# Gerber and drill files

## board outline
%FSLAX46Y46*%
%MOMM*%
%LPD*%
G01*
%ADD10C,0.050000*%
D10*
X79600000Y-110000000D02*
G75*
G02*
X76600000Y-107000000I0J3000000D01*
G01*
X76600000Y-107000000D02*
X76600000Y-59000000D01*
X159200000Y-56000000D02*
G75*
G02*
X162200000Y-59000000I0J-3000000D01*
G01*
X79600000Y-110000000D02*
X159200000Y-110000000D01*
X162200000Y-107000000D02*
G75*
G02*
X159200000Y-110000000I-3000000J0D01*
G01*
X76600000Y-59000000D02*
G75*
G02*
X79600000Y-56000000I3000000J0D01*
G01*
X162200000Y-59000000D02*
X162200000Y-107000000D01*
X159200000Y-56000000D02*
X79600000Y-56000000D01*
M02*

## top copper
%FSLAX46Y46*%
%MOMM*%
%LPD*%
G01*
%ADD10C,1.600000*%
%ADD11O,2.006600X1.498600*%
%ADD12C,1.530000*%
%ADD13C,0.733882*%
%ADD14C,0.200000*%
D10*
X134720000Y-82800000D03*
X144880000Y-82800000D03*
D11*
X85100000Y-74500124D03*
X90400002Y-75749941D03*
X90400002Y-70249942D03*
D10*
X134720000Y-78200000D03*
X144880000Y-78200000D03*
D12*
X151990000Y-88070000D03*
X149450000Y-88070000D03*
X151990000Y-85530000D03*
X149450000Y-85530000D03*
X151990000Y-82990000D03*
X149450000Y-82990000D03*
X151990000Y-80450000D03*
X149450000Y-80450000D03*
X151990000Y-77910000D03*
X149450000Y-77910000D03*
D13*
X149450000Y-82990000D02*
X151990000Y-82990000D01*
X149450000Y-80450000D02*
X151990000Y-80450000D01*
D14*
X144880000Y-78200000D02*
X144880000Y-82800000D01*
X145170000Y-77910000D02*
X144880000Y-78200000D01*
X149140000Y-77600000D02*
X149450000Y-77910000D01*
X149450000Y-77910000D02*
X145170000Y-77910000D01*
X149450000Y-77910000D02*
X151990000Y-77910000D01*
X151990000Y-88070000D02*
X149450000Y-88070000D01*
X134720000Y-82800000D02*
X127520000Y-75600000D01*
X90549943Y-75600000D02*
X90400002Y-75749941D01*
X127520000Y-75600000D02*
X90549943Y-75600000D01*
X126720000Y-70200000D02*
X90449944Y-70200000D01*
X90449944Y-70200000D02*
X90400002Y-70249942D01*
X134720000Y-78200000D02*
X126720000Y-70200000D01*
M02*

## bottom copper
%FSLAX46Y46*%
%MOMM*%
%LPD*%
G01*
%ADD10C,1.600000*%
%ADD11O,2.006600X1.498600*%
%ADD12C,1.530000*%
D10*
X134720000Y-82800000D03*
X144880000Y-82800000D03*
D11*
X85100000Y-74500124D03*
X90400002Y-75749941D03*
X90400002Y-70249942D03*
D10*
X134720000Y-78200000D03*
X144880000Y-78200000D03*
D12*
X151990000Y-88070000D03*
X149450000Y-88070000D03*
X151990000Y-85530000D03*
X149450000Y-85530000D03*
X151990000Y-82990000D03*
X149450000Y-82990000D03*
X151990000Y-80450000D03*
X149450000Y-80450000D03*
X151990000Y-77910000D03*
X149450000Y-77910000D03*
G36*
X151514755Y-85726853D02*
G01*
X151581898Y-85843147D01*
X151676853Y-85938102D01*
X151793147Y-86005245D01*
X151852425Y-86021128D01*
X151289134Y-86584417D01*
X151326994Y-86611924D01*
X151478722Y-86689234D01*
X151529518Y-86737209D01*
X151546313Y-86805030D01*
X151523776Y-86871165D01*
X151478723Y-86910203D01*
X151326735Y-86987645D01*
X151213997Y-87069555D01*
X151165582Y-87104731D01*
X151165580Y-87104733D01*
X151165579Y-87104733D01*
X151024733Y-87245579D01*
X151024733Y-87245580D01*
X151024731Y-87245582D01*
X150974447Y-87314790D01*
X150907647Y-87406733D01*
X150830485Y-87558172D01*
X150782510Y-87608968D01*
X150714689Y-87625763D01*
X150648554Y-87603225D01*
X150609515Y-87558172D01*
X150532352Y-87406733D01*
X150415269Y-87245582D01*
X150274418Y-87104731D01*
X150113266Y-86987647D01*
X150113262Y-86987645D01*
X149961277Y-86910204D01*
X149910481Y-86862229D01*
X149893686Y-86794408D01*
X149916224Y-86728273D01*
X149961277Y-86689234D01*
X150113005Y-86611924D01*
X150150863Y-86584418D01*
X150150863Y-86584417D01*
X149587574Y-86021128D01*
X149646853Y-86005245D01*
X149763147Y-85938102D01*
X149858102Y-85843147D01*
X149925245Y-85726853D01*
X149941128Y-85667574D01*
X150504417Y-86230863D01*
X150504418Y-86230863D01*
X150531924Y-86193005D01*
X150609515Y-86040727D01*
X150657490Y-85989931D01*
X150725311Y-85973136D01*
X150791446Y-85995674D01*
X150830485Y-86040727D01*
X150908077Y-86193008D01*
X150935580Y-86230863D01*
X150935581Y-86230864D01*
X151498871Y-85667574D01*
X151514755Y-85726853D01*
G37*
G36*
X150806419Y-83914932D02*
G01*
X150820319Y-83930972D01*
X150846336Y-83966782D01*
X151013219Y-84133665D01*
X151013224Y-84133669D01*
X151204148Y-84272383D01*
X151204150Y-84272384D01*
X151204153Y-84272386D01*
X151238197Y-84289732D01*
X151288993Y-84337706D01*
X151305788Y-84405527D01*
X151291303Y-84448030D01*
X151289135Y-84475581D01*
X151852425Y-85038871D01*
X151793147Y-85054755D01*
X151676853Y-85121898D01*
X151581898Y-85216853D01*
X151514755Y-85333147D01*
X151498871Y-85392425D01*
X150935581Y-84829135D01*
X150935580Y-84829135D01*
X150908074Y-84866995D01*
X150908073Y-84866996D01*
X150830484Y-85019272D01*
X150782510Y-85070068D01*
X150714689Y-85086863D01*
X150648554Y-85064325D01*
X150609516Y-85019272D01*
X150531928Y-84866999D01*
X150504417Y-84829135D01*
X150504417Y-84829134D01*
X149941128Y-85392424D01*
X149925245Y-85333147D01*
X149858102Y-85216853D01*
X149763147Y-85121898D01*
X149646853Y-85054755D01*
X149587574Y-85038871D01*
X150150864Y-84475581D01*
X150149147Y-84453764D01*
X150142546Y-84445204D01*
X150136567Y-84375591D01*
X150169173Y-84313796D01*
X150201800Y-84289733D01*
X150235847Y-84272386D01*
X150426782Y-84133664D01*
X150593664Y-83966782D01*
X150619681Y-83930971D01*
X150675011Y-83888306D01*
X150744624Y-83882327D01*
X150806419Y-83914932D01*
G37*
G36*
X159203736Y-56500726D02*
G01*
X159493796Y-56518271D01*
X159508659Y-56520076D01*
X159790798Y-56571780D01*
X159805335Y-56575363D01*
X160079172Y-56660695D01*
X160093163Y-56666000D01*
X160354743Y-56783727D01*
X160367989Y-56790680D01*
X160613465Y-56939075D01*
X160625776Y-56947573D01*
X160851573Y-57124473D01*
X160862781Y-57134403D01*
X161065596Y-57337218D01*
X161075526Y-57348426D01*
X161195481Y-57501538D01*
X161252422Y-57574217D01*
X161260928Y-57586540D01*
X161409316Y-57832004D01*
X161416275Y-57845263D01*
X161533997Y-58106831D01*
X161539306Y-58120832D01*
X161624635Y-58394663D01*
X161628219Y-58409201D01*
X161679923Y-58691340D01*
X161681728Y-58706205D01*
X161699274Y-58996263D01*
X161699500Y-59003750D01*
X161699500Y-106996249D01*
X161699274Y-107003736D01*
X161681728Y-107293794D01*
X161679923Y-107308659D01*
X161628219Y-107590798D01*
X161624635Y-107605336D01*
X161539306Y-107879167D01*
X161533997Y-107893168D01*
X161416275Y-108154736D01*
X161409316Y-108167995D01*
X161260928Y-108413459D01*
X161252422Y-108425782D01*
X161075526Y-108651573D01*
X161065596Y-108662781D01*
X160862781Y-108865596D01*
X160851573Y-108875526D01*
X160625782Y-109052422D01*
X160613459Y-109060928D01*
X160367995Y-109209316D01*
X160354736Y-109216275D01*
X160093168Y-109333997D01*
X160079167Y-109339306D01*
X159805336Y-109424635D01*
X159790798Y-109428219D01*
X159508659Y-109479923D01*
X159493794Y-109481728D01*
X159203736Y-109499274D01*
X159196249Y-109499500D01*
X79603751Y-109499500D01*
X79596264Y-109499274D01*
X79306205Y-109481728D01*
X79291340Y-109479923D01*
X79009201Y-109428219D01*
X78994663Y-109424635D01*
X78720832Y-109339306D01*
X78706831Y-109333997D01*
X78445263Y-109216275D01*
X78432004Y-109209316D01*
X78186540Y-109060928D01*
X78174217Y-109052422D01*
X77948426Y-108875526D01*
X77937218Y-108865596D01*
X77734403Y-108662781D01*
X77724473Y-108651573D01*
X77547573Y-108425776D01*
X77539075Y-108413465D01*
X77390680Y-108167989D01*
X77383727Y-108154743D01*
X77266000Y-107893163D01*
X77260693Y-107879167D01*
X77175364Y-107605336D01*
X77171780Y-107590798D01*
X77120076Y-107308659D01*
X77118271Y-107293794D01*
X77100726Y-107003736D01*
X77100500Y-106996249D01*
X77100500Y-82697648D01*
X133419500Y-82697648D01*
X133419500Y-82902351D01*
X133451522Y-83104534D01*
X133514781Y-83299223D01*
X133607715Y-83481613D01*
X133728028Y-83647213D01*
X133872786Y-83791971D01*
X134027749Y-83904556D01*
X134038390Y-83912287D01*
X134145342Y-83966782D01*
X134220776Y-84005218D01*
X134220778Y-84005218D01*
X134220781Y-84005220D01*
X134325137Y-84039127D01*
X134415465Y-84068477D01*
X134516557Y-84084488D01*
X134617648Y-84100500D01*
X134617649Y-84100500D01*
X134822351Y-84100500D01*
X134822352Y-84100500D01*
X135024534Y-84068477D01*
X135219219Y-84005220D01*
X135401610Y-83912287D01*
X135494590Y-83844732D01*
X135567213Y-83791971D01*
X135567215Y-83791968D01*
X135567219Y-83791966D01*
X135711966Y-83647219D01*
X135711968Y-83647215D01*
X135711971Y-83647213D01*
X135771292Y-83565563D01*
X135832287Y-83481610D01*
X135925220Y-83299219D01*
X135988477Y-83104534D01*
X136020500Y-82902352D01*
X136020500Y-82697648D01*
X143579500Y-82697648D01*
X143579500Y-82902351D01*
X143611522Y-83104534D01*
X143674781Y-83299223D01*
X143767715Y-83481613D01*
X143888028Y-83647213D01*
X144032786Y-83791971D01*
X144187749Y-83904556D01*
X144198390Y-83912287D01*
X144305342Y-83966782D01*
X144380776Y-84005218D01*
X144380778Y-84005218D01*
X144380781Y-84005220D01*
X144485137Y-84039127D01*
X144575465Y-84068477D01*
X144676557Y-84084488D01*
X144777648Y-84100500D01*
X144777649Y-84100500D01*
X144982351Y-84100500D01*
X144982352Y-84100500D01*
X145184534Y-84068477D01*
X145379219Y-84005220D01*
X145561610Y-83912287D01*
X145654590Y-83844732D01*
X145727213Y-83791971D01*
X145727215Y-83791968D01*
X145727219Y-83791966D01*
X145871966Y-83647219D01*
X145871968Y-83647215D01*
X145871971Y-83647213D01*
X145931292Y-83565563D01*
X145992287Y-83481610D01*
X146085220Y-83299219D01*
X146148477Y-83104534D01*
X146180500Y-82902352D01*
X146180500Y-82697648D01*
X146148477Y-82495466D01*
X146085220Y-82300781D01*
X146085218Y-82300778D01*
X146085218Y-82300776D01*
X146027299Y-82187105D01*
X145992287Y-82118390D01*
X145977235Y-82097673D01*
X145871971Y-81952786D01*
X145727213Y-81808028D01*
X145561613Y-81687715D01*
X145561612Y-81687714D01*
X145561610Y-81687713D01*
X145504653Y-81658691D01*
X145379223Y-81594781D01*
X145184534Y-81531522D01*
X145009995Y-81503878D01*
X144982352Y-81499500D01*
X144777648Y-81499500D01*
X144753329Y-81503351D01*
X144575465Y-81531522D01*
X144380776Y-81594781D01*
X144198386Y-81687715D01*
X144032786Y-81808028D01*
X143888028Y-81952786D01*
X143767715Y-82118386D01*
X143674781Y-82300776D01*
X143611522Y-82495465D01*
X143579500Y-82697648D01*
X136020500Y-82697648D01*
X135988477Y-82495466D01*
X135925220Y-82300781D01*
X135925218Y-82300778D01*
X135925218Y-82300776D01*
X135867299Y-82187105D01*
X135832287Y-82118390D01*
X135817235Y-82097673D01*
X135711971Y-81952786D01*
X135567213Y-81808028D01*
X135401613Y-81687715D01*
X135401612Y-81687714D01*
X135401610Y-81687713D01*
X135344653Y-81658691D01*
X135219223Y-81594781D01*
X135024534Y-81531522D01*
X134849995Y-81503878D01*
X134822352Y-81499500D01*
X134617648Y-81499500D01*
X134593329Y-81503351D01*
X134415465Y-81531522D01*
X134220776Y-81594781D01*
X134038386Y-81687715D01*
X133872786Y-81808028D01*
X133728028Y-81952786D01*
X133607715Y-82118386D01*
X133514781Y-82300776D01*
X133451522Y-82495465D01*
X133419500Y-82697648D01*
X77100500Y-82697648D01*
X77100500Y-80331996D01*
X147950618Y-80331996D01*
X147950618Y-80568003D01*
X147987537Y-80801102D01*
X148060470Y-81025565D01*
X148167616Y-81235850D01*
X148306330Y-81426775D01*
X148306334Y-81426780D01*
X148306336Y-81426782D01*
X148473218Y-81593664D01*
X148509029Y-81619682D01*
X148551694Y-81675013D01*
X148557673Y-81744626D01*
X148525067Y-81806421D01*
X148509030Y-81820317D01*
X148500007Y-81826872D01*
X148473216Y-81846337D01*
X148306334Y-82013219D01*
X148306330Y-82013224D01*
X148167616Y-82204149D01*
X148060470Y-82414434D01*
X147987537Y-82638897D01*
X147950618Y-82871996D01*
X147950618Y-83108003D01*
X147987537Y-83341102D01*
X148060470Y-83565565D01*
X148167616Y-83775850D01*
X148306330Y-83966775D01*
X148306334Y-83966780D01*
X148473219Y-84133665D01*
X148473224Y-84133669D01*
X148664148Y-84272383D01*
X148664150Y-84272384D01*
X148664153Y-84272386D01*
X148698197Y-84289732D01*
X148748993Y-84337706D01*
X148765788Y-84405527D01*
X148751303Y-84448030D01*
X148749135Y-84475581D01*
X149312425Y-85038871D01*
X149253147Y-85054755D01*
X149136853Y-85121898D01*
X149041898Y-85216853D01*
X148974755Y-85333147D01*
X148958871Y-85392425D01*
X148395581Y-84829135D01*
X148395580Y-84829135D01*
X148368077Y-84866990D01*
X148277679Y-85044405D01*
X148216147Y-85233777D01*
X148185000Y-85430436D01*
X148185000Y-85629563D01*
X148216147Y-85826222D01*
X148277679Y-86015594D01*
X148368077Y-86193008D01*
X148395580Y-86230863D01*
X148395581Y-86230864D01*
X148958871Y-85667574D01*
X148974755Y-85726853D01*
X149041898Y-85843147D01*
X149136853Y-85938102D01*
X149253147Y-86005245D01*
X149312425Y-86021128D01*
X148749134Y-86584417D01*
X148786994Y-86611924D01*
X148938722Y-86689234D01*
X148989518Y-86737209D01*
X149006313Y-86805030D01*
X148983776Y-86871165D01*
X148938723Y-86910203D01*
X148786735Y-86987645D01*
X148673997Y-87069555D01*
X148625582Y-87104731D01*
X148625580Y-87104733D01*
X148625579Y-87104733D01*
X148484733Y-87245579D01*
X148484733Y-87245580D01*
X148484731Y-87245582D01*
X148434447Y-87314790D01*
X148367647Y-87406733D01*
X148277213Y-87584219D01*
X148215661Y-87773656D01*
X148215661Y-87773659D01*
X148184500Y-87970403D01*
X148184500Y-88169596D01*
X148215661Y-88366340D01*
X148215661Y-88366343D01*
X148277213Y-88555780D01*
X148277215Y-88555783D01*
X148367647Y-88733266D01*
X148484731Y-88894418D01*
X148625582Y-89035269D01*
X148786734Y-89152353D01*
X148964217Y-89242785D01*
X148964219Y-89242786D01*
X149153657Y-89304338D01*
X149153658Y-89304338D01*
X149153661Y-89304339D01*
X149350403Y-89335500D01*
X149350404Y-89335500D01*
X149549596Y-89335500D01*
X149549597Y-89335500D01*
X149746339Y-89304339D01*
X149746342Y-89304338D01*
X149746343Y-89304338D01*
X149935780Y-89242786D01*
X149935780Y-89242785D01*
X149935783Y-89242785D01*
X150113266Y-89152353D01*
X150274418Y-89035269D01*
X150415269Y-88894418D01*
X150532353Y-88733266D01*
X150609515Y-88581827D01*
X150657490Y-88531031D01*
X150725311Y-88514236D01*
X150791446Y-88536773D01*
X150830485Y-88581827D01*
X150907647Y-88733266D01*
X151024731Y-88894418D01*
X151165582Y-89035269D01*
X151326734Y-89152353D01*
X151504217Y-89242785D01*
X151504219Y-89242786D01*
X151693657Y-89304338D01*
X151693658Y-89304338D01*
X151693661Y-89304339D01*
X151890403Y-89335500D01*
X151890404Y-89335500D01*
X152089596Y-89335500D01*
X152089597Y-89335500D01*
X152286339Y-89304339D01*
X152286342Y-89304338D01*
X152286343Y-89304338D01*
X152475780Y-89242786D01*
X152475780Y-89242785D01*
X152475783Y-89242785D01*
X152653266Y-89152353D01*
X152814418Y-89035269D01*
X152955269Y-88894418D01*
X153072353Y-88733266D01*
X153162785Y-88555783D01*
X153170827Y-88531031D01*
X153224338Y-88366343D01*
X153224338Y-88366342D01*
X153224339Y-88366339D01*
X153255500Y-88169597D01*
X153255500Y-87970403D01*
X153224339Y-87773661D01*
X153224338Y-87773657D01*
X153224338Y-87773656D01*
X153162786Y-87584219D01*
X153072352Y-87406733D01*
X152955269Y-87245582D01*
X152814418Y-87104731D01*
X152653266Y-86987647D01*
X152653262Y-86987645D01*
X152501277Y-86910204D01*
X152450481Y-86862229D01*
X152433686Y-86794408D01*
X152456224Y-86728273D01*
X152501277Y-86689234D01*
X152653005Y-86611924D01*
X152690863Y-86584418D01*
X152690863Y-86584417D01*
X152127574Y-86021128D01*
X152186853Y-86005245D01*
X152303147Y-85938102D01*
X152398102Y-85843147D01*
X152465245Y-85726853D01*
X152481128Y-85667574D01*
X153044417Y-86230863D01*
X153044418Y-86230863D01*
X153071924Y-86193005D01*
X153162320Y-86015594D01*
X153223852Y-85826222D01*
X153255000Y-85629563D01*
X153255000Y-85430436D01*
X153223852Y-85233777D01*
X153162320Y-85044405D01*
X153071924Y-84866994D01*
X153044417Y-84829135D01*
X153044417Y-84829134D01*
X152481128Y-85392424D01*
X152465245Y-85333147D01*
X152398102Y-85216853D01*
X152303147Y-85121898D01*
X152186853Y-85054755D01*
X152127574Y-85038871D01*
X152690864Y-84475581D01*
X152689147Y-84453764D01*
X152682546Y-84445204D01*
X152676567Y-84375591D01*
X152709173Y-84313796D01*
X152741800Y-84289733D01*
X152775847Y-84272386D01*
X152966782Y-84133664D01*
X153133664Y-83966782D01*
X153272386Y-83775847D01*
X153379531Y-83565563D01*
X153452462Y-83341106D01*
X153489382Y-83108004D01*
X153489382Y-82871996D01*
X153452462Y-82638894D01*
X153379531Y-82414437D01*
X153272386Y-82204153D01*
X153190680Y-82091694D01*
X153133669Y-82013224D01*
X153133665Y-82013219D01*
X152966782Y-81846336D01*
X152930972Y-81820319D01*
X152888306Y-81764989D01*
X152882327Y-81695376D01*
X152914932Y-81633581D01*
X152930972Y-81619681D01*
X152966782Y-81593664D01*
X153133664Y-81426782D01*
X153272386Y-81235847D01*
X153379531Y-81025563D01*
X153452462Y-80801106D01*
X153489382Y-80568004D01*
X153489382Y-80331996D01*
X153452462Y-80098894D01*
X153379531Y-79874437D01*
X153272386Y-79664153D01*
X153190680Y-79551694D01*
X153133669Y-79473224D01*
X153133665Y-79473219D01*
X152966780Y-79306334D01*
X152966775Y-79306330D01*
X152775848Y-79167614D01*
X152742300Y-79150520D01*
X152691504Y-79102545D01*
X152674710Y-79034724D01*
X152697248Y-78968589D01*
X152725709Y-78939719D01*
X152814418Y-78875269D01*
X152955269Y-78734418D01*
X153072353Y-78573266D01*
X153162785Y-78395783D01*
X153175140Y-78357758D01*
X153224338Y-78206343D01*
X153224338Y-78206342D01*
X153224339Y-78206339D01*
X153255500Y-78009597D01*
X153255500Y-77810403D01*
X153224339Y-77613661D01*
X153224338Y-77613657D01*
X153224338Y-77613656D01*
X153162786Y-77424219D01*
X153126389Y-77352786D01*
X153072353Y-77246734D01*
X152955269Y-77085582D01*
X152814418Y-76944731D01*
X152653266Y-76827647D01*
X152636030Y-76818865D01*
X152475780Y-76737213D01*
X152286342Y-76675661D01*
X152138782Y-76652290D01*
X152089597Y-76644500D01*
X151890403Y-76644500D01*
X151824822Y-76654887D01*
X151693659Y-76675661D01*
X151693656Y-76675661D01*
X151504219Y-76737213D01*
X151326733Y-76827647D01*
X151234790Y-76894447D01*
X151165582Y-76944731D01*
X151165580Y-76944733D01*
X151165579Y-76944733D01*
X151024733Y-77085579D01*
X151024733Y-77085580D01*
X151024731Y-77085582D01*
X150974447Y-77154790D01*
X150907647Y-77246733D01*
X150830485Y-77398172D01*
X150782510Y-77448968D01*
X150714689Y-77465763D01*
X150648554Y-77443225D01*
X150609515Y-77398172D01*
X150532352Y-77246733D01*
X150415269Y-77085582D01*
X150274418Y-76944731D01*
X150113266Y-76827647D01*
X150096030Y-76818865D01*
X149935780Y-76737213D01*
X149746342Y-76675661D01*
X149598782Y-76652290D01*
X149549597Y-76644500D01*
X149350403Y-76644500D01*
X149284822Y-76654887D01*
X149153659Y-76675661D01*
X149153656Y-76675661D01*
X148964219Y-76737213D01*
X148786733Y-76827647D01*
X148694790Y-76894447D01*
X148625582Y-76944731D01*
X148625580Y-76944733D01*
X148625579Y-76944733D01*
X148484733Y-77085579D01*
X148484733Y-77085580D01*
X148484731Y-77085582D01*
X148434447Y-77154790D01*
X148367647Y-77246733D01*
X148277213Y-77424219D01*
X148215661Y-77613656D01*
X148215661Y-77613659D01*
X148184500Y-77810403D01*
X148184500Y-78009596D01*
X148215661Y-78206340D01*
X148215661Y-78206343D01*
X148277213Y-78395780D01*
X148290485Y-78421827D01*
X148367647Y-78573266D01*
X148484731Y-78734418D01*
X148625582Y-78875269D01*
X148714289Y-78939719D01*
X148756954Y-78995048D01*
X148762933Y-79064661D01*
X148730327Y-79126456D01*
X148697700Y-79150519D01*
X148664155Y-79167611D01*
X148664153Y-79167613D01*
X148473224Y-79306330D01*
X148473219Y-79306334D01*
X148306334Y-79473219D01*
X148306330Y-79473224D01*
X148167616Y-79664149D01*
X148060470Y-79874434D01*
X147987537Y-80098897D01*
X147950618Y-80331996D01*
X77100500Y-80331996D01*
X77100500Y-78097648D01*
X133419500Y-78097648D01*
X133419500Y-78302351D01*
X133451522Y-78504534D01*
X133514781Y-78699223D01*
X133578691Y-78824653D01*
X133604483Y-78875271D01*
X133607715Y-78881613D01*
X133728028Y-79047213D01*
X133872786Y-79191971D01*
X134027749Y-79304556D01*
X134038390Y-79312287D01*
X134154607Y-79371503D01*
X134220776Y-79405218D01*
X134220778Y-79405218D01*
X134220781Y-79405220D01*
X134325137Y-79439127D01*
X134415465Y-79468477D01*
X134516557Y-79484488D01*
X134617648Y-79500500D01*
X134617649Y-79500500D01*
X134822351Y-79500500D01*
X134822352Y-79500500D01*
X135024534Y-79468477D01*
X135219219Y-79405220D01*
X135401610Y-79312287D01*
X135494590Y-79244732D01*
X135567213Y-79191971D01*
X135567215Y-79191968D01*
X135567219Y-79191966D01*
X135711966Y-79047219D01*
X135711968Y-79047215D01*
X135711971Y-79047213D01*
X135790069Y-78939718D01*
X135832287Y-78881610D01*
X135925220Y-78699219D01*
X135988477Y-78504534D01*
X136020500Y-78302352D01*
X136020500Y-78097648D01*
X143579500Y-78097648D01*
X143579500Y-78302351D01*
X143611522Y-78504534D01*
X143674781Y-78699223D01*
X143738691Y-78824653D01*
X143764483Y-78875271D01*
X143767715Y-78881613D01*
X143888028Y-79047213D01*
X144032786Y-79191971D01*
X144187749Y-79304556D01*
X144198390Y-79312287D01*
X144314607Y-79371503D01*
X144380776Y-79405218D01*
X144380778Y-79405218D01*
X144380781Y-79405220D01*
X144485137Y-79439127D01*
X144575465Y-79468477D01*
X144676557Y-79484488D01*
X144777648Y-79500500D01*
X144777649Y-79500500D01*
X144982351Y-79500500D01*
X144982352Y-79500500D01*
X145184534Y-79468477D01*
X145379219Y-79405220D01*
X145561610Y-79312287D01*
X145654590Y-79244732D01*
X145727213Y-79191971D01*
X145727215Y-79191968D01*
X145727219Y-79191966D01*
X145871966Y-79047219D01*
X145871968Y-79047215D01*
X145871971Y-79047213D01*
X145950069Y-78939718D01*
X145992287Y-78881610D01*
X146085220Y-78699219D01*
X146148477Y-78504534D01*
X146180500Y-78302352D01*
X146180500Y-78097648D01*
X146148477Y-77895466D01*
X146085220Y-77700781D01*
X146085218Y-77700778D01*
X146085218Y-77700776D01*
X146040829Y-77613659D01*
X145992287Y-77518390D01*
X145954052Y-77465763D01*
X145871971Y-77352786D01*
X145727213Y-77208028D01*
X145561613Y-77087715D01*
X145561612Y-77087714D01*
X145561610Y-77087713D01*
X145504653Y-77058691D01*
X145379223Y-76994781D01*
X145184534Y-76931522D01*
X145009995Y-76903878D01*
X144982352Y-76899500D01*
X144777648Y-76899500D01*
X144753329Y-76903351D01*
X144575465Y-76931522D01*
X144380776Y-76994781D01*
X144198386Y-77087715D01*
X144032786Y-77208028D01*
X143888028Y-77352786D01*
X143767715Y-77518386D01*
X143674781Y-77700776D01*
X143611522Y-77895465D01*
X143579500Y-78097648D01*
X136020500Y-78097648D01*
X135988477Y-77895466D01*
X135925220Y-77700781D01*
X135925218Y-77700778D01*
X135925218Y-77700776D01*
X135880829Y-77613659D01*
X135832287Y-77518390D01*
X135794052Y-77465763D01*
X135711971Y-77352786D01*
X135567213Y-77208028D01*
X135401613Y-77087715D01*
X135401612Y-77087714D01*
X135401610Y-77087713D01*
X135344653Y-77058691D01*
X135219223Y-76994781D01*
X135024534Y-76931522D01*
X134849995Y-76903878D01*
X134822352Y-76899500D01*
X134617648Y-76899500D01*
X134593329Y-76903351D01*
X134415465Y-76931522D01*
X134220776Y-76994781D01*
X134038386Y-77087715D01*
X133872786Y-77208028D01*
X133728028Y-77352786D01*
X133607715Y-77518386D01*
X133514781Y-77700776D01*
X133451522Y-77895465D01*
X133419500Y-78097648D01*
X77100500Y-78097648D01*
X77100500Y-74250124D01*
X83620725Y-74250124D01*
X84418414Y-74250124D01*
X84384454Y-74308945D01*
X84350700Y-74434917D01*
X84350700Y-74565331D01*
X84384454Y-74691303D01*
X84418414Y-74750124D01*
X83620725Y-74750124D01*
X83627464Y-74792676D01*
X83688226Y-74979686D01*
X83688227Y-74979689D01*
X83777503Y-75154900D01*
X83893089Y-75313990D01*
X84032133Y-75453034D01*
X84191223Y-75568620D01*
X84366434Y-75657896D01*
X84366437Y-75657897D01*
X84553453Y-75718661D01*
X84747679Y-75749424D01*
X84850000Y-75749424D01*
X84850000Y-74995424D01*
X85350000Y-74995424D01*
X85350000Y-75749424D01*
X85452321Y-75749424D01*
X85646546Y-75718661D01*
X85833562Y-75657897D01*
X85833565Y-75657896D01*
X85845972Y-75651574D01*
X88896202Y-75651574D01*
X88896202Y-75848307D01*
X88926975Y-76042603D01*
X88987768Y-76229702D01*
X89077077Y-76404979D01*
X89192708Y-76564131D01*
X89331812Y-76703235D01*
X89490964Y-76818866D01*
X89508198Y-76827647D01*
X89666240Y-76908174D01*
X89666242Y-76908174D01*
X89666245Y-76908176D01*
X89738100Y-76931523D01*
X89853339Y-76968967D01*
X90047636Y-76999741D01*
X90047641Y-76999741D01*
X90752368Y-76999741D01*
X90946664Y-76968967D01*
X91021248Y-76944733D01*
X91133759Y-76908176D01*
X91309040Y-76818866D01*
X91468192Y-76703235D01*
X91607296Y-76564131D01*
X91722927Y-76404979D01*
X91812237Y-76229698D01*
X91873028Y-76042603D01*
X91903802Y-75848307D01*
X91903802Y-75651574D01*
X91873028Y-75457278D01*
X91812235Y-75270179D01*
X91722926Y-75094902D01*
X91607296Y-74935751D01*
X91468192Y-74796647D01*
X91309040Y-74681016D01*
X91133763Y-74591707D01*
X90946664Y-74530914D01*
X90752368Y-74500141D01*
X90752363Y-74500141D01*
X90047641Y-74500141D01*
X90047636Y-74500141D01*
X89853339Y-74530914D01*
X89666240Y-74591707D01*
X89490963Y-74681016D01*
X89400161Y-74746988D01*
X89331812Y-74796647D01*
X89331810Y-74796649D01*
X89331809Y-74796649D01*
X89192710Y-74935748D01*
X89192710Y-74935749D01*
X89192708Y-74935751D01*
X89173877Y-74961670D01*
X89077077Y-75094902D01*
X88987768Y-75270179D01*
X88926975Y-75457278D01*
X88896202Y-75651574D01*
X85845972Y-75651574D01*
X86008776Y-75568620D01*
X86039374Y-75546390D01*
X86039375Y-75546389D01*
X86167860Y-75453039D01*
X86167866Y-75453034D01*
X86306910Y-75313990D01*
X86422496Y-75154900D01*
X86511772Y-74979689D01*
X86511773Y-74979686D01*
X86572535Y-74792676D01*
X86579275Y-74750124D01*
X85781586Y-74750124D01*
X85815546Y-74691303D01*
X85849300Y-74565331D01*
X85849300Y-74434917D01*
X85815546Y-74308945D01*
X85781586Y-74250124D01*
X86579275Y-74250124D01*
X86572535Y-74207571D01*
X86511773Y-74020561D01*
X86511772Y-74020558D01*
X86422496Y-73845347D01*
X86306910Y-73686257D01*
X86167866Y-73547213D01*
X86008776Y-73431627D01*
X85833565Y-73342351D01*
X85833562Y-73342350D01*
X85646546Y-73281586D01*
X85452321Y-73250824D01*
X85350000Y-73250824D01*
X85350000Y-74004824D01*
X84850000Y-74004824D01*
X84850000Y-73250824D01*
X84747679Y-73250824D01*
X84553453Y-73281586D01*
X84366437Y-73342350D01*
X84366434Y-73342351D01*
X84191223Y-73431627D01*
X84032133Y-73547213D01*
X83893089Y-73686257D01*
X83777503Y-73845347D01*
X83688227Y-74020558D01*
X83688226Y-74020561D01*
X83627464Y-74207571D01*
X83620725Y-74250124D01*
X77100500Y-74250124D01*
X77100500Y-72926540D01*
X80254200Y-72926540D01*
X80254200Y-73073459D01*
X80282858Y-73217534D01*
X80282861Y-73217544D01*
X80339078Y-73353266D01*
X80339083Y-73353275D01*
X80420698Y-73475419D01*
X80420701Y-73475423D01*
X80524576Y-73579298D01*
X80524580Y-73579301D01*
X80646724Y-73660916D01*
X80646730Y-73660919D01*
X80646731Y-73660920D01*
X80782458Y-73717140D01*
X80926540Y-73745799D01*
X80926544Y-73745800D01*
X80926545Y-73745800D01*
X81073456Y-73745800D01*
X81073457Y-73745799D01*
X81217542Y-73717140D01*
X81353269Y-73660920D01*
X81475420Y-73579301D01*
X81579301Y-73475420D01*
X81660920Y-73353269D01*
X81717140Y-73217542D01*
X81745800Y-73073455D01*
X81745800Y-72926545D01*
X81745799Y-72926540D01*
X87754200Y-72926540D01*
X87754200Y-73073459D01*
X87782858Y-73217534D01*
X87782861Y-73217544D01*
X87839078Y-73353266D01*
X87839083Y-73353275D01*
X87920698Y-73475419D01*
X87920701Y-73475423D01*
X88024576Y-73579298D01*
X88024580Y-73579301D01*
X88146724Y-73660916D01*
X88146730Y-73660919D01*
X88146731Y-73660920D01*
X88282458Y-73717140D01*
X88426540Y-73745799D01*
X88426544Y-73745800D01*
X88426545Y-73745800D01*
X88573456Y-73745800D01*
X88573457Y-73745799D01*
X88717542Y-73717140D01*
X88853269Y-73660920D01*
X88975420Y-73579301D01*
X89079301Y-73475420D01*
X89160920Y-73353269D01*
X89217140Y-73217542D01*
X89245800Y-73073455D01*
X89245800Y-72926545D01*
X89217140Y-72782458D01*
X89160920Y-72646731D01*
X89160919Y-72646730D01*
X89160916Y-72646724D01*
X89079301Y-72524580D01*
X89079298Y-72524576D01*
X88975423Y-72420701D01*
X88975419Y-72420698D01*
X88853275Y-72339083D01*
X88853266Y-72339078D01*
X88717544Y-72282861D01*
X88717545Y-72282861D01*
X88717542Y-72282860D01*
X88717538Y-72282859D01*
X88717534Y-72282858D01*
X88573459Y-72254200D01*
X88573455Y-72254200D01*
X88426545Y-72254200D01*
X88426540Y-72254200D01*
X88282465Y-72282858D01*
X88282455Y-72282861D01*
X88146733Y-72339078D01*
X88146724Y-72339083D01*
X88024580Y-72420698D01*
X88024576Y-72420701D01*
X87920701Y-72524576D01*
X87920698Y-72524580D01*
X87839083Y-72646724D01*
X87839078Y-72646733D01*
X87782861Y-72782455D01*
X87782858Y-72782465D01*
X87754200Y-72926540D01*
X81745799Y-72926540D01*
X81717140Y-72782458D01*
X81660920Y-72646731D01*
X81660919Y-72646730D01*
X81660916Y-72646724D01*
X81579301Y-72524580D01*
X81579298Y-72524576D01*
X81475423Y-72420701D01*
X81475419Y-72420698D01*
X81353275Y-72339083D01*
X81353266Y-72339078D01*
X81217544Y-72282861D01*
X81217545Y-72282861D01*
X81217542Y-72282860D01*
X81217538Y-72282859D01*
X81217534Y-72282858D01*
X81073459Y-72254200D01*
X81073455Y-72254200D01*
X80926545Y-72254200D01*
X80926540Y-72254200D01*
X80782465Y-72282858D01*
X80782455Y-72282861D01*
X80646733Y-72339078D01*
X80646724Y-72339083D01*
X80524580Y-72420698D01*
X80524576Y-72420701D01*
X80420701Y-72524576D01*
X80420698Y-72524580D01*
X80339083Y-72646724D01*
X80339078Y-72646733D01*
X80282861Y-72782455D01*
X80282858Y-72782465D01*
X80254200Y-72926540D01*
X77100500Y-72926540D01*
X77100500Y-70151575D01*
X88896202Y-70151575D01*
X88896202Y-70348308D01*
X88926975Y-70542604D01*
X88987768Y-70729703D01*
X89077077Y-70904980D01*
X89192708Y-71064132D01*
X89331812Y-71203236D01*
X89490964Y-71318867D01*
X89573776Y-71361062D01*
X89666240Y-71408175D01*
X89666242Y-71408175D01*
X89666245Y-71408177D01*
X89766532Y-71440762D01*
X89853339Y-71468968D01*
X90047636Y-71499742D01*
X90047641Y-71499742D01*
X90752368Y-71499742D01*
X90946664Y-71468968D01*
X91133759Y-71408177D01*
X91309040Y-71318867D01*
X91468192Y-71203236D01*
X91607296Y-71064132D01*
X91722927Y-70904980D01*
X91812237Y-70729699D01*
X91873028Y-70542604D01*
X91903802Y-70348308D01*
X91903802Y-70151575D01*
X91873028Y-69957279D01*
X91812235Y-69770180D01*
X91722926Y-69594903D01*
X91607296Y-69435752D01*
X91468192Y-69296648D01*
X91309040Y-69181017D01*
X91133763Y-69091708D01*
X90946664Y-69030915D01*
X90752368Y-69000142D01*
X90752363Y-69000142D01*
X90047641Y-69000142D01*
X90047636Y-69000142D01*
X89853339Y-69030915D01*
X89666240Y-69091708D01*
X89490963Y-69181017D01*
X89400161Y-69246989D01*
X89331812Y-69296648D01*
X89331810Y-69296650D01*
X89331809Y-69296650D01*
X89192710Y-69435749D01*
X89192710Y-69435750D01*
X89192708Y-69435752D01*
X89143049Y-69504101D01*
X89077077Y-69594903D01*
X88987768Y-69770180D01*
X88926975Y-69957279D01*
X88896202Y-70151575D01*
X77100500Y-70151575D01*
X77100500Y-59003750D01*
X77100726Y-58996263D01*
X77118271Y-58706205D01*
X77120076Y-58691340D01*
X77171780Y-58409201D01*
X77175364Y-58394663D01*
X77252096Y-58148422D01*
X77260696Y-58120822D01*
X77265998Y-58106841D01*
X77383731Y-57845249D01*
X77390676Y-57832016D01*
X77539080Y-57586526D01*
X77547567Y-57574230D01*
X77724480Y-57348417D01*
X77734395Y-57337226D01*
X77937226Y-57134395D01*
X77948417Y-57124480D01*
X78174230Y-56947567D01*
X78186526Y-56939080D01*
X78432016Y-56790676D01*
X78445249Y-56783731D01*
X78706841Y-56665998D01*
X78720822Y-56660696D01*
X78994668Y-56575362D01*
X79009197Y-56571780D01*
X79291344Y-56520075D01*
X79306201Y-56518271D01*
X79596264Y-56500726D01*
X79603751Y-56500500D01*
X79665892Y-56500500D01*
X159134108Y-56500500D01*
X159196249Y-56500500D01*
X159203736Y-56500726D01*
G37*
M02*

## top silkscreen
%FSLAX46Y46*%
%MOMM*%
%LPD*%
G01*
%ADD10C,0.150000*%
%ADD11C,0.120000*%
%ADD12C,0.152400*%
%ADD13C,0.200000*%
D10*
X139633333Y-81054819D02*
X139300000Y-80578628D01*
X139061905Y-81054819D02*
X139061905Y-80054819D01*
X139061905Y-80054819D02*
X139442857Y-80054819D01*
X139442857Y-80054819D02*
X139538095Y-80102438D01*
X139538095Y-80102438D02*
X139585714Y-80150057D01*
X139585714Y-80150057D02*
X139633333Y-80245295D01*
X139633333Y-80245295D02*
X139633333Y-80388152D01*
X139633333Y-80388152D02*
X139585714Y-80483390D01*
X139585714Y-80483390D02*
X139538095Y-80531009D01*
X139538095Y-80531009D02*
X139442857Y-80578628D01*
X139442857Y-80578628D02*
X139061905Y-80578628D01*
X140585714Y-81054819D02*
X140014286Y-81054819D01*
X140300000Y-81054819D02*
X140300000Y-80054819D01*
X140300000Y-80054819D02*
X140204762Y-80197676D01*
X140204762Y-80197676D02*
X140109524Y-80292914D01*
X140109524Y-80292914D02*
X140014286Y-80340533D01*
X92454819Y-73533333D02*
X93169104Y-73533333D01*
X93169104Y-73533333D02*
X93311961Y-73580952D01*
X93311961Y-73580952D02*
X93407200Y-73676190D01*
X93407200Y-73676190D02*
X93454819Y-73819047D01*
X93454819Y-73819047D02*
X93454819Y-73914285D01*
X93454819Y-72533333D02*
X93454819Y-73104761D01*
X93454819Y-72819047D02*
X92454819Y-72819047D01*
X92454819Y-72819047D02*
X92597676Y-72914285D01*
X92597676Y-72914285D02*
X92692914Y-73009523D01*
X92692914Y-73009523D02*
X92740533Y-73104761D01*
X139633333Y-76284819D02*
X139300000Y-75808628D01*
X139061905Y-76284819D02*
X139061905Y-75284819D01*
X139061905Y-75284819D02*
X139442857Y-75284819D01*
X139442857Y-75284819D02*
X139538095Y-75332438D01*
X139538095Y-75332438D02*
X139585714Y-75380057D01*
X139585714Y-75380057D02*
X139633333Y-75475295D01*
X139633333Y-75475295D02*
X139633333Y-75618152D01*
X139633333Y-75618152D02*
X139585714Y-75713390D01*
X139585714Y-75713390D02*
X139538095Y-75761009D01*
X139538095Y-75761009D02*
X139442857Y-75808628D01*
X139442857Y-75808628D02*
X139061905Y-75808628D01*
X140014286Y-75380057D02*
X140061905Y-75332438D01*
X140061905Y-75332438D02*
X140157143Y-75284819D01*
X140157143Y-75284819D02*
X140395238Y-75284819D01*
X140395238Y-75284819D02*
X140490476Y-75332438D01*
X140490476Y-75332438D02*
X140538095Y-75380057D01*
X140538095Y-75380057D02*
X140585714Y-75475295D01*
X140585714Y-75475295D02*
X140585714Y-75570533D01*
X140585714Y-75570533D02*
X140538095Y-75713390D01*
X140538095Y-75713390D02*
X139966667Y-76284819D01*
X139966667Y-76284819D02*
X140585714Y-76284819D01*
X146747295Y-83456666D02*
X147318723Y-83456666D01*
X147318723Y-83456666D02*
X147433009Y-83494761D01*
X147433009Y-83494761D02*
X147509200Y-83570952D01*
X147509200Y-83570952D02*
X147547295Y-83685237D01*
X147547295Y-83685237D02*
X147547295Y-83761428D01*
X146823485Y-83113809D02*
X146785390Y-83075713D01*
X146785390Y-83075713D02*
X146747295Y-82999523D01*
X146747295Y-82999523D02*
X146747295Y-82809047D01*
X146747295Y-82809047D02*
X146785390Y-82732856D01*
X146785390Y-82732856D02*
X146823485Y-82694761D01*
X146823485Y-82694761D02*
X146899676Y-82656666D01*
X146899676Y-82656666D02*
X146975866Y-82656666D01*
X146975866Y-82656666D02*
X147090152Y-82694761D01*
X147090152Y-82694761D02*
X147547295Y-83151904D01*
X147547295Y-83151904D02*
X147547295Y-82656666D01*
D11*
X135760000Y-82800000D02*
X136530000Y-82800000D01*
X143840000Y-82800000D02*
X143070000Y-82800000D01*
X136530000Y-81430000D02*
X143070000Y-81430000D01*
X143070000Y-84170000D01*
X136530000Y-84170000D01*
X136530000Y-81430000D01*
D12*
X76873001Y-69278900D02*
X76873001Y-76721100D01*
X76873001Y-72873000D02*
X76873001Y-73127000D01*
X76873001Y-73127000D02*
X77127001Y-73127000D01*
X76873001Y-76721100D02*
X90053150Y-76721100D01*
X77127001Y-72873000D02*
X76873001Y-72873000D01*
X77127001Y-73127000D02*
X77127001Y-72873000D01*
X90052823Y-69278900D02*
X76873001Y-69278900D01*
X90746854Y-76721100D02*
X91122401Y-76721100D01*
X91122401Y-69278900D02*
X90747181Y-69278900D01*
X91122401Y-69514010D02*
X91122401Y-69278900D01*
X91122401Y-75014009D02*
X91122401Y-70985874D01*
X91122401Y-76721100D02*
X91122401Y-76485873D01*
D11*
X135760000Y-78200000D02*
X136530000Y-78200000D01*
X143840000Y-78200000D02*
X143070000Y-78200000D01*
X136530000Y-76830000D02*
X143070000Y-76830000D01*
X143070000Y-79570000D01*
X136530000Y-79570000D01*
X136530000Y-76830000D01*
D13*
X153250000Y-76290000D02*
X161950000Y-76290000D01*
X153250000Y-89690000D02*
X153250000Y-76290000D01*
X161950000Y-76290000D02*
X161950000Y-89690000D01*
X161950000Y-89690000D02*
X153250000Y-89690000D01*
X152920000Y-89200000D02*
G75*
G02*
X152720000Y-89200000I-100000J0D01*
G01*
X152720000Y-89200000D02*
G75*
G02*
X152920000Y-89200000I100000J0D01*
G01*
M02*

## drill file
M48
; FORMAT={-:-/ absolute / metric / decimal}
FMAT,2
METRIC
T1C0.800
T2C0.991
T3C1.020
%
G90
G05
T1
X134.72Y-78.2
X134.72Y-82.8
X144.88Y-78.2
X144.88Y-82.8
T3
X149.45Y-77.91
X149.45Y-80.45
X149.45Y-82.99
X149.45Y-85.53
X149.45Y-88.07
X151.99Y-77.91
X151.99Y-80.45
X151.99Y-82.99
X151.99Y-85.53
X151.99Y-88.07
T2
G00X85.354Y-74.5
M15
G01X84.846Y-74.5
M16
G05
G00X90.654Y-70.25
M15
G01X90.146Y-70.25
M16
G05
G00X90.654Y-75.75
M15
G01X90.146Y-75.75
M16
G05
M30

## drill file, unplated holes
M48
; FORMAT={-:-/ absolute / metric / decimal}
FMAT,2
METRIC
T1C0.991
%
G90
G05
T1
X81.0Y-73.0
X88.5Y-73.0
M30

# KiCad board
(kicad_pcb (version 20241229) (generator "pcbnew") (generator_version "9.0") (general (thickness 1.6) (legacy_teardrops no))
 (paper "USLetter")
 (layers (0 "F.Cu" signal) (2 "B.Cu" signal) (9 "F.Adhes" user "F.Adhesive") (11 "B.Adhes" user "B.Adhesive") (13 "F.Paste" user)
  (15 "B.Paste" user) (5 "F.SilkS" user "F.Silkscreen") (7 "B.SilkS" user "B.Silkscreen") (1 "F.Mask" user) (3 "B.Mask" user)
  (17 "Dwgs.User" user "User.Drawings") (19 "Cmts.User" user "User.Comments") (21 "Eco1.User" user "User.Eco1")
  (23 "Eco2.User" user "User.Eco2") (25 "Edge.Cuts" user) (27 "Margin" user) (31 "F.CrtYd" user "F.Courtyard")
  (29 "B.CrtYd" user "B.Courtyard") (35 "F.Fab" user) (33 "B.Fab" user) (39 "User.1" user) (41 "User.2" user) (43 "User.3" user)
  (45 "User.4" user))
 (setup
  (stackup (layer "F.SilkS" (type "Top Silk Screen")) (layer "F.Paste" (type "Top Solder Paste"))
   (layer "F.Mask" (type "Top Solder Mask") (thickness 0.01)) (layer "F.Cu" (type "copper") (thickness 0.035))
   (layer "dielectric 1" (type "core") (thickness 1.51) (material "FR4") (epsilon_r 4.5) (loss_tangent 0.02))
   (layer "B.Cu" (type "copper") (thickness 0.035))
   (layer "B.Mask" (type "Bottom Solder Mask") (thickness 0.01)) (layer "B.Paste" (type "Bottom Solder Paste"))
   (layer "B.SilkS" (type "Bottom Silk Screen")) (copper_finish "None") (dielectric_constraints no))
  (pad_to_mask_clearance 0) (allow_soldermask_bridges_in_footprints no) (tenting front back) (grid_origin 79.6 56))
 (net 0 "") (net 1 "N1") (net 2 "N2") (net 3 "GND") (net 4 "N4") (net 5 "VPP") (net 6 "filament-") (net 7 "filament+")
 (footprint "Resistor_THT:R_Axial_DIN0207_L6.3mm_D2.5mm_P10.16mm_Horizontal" (layer "F.Cu") (at 134.72 82.8)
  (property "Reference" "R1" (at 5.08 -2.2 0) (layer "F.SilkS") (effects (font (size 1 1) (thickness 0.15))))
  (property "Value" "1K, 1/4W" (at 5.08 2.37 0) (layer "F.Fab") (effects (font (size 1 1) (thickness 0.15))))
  (fp_line (start 1.04 0) (end 1.81 0) (stroke (width 0.12) (type solid)) (layer "F.SilkS"))
  (fp_line (start 9.12 0) (end 8.35 0) (stroke (width 0.12) (type solid)) (layer "F.SilkS"))
  (fp_rect (start 1.81 -1.37) (end 8.35 1.37) (stroke (width 0.12) (type solid)) (fill no) (layer "F.SilkS"))
  (pad "1" thru_hole circle (at 0 0) (size 1.6 1.6) (drill 0.8) (layers "*.Cu" "*.Mask") (remove_unused_layers no) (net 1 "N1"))
  (pad "2" thru_hole circle (at 10.16 0) (size 1.6 1.6) (drill 0.8) (layers "*.Cu" "*.Mask") (remove_unused_layers no) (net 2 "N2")))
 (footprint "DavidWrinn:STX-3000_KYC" (layer "F.Cu") (at 85.1 74.500124 90)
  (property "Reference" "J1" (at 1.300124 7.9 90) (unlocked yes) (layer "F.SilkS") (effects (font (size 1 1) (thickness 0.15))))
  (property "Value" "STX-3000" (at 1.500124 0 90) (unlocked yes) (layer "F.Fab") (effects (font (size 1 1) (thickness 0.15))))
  (fp_line (start 5.221224 -8.226999) (end -2.220976 -8.226999) (stroke (width 0.1524) (type solid)) (layer "F.SilkS"))
  (fp_line (start 1.627124 -8.226999) (end 1.373124 -8.226999) (stroke (width 0.1524) (type solid)) (layer "F.SilkS"))
  (fp_line (start 1.373124 -8.226999) (end 1.373124 -7.972999) (stroke (width 0.1524) (type solid)) (layer "F.SilkS"))
  (fp_line (start -2.220976 -8.226999) (end -2.220976 4.95315) (stroke (width 0.1524) (type solid)) (layer "F.SilkS"))
  (fp_line (start 1.627124 -7.972999) (end 1.627124 -8.226999) (stroke (width 0.1524) (type solid)) (layer "F.SilkS"))
  (fp_line (start 1.373124 -7.972999) (end 1.627124 -7.972999) (stroke (width 0.1524) (type solid)) (layer "F.SilkS"))
  (fp_line (start 5.221224 4.952823) (end 5.221224 -8.226999) (stroke (width 0.1524) (type solid)) (layer "F.SilkS"))
  (fp_line (start -2.220976 5.646854) (end -2.220976 6.022401) (stroke (width 0.1524) (type solid)) (layer "F.SilkS"))
  (fp_line (start 5.221224 6.022401) (end 5.221224 5.647181) (stroke (width 0.1524) (type solid)) (layer "F.SilkS"))
  (fp_line (start 4.986114 6.022401) (end 5.221224 6.022401) (stroke (width 0.1524) (type solid)) (layer "F.SilkS"))
  (fp_line (start -0.513885 6.022401) (end 3.51425 6.022401) (stroke (width 0.1524) (type solid)) (layer "F.SilkS"))
  (fp_line (start -2.220976 6.022401) (end -1.985749 6.022401) (stroke (width 0.1524) (type solid)) (layer "F.SilkS"))
  (pad "" np_thru_hole circle (at 1.500124 -4.1 90) (size 0.9906 0.9906) (drill 0.9906) (layers "*.Cu" "*.Mask"))
  (pad "" np_thru_hole circle (at 1.500124 3.4 90) (size 0.9906 0.9906) (drill 0.9906) (layers "*.Cu" "*.Mask"))
  (pad "1" thru_hole oval (at 0 0 180) (size 2.0066 1.4986) (drill oval 1.4986 0.9906) (layers "*.Cu" "*.Mask") (remove_unused_layers no)
   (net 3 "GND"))
  (pad "2" thru_hole oval (at -1.249817 5.300002 180) (size 2.0066 1.4986) (drill oval 1.4986 0.9906) (layers "*.Cu" "*.Mask")
   (remove_unused_layers no) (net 1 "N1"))
  (pad "3" thru_hole oval (at 4.250182 5.300002 180) (size 2.0066 1.4986) (drill oval 1.4986 0.9906) (layers "*.Cu" "*.Mask")
   (remove_unused_layers no) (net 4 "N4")))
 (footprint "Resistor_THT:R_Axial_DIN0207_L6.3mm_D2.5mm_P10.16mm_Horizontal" (layer "F.Cu") (at 134.72 78.2)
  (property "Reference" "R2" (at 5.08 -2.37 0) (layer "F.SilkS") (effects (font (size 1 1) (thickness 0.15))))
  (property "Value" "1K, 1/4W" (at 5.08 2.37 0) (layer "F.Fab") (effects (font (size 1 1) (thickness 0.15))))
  (fp_line (start 1.04 0) (end 1.81 0) (stroke (width 0.12) (type solid)) (layer "F.SilkS"))
  (fp_line (start 9.12 0) (end 8.35 0) (stroke (width 0.12) (type solid)) (layer "F.SilkS"))
  (fp_rect (start 1.81 -1.37) (end 8.35 1.37) (stroke (width 0.12) (type solid)) (fill no) (layer "F.SilkS"))
  (pad "1" thru_hole circle (at 0 0) (size 1.6 1.6) (drill 0.8) (layers "*.Cu" "*.Mask") (remove_unused_layers no) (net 4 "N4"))
  (pad "2" thru_hole circle (at 10.16 0) (size 1.6 1.6) (drill 0.8) (layers "*.Cu" "*.Mask") (remove_unused_layers no) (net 2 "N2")))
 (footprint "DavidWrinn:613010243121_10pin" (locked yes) (layer "F.Cu") (at 157.6 82.99 90)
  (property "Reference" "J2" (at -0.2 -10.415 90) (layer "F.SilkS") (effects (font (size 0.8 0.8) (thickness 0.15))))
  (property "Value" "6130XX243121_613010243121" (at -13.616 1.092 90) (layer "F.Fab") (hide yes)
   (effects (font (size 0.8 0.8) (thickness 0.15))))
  (fp_line (start 6.7 -4.35) (end 6.7 4.35) (stroke (width 0.2) (type solid)) (layer "F.SilkS"))
  (fp_line (start -6.7 -4.35) (end 6.7 -4.35) (stroke (width 0.2) (type solid)) (layer "F.SilkS"))
  (fp_line (start 6.7 4.35) (end -6.7 4.35) (stroke (width 0.2) (type solid)) (layer "F.SilkS"))
  (fp_line (start -6.7 4.35) (end -6.7 -4.35) (stroke (width 0.2) (type solid)) (layer "F.SilkS"))
  (fp_circle (center -6.21 -4.78) (end -6.11 -4.78) (stroke (width 0.2) (type solid)) (fill no) (layer "F.SilkS"))
  (pad "1" thru_hole circle (at -5.08 -5.61 90) (size 1.53 1.53) (drill 1.02) (layers "*.Cu" "*.Mask") (remove_unused_layers no)
   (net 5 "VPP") (solder_mask_margin 0.102))
  (pad "2" thru_hole circle (at -5.08 -8.15 90) (size 1.53 1.53) (drill 1.02) (layers "*.Cu" "*.Mask") (remove_unused_layers no)
   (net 5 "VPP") (solder_mask_margin 0.102))
  (pad "3" thru_hole circle (at -2.54 -5.61 90) (size 1.53 1.53) (drill 1.02) (layers "*.Cu" "*.Mask") (remove_unused_layers no)
   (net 3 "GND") (solder_mask_margin 0.102))
  (pad "4" thru_hole circle (at -2.54 -8.15 90) (size 1.53 1.53) (drill 1.02) (layers "*.Cu" "*.Mask") (remove_unused_layers no)
   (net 3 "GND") (solder_mask_margin 0.102))
  (pad "5" thru_hole circle (at 0 -5.61 90) (size 1.53 1.53) (drill 1.02) (layers "*.Cu" "*.Mask") (remove_unused_layers no)
   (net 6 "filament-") (solder_mask_margin 0.102))
  (pad "6" thru_hole circle (at 0 -8.15 90) (size 1.53 1.53) (drill 1.02) (layers "*.Cu" "*.Mask") (remove_unused_layers no)
   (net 6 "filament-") (solder_mask_margin 0.102))
  (pad "7" thru_hole circle (at 2.54 -5.61 90) (size 1.53 1.53) (drill 1.02) (layers "*.Cu" "*.Mask") (remove_unused_layers no)
   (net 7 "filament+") (solder_mask_margin 0.102))
  (pad "8" thru_hole circle (at 2.54 -8.15 90) (size 1.53 1.53) (drill 1.02) (layers "*.Cu" "*.Mask") (remove_unused_layers no)
   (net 7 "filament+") (solder_mask_margin 0.102))
  (pad "9" thru_hole circle (at 5.08 -5.61 90) (size 1.53 1.53) (drill 1.02) (layers "*.Cu" "*.Mask") (remove_unused_layers no) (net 2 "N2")
   (solder_mask_margin 0.102))
  (pad "10" thru_hole circle (at 5.08 -8.15 90) (size 1.53 1.53) (drill 1.02) (layers "*.Cu" "*.Mask") (remove_unused_layers no)
   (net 2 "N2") (solder_mask_margin 0.102)))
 (gr_arc (start 79.6 110) (mid 77.47868 109.12132) (end 76.6 107) (stroke (width 0.05) (type default)) (layer "Edge.Cuts"))
 (gr_line (start 76.6 107) (end 76.6 59) (stroke (width 0.05) (type default)) (layer "Edge.Cuts"))
 (gr_arc (start 159.2 56) (mid 161.32132 56.87868) (end 162.2 59) (stroke (width 0.05) (type default)) (layer "Edge.Cuts"))
 (gr_line (start 79.6 110) (end 159.2 110) (stroke (width 0.05) (type default)) (layer "Edge.Cuts"))
 (gr_arc (start 162.2 107) (mid 161.32132 109.12132) (end 159.2 110) (stroke (width 0.05) (type default)) (layer "Edge.Cuts"))
 (gr_arc (start 76.6 59) (mid 77.47868 56.87868) (end 79.6 56) (stroke (width 0.05) (type default)) (layer "Edge.Cuts"))
 (gr_line (start 162.2 59) (end 162.2 107) (stroke (width 0.05) (type default)) (layer "Edge.Cuts"))
 (gr_line (start 159.2 56) (end 79.6 56) (stroke (width 0.05) (type default)) (layer "Edge.Cuts"))
 (segment (start 149.45 80.45) (end 151.99 80.45) (width 0.733882) (layer "F.Cu") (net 7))
 (segment (start 144.88 78.2) (end 144.88 82.8) (width 0.2) (layer "F.Cu") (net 2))
 (segment (start 145.17 77.91) (end 144.88 78.2) (width 0.2) (layer "F.Cu") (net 2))
 (segment (start 149.14 77.6) (end 149.45 77.91) (width 0.2) (layer "F.Cu") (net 2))
 (segment (start 149.45 77.91) (end 145.17 77.91) (width 0.2) (layer "F.Cu") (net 2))
 (segment (start 149.45 77.91) (end 151.99 77.91) (width 0.2) (layer "F.Cu") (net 2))
 (segment (start 151.99 88.07) (end 149.45 88.07) (width 0.2) (layer "F.Cu") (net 5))
 (segment (start 149.45 82.99) (end 151.99 82.99) (width 0.733882) (layer "F.Cu") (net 6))
 (segment (start 134.72 82.8) (end 127.52 75.6) (width 0.2) (layer "F.Cu") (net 1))
 (segment (start 90.549943 75.6) (end 90.400002 75.749941) (width 0.2) (layer "F.Cu") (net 1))
 (segment (start 127.52 75.6) (end 90.549943 75.6) (width 0.2) (layer "F.Cu") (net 1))
 (segment (start 126.72 70.2) (end 90.449944 70.2) (width 0.2) (layer "F.Cu") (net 4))
 (segment (start 90.449944 70.2) (end 90.400002 70.249942) (width 0.2) (layer "F.Cu") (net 4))
 (segment (start 134.72 78.2) (end 126.72 70.2) (width 0.2) (layer "F.Cu") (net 4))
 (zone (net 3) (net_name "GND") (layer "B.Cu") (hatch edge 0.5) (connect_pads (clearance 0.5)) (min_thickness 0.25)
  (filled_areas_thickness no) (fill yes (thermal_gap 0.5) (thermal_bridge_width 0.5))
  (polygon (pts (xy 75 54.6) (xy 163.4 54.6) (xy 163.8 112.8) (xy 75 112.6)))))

